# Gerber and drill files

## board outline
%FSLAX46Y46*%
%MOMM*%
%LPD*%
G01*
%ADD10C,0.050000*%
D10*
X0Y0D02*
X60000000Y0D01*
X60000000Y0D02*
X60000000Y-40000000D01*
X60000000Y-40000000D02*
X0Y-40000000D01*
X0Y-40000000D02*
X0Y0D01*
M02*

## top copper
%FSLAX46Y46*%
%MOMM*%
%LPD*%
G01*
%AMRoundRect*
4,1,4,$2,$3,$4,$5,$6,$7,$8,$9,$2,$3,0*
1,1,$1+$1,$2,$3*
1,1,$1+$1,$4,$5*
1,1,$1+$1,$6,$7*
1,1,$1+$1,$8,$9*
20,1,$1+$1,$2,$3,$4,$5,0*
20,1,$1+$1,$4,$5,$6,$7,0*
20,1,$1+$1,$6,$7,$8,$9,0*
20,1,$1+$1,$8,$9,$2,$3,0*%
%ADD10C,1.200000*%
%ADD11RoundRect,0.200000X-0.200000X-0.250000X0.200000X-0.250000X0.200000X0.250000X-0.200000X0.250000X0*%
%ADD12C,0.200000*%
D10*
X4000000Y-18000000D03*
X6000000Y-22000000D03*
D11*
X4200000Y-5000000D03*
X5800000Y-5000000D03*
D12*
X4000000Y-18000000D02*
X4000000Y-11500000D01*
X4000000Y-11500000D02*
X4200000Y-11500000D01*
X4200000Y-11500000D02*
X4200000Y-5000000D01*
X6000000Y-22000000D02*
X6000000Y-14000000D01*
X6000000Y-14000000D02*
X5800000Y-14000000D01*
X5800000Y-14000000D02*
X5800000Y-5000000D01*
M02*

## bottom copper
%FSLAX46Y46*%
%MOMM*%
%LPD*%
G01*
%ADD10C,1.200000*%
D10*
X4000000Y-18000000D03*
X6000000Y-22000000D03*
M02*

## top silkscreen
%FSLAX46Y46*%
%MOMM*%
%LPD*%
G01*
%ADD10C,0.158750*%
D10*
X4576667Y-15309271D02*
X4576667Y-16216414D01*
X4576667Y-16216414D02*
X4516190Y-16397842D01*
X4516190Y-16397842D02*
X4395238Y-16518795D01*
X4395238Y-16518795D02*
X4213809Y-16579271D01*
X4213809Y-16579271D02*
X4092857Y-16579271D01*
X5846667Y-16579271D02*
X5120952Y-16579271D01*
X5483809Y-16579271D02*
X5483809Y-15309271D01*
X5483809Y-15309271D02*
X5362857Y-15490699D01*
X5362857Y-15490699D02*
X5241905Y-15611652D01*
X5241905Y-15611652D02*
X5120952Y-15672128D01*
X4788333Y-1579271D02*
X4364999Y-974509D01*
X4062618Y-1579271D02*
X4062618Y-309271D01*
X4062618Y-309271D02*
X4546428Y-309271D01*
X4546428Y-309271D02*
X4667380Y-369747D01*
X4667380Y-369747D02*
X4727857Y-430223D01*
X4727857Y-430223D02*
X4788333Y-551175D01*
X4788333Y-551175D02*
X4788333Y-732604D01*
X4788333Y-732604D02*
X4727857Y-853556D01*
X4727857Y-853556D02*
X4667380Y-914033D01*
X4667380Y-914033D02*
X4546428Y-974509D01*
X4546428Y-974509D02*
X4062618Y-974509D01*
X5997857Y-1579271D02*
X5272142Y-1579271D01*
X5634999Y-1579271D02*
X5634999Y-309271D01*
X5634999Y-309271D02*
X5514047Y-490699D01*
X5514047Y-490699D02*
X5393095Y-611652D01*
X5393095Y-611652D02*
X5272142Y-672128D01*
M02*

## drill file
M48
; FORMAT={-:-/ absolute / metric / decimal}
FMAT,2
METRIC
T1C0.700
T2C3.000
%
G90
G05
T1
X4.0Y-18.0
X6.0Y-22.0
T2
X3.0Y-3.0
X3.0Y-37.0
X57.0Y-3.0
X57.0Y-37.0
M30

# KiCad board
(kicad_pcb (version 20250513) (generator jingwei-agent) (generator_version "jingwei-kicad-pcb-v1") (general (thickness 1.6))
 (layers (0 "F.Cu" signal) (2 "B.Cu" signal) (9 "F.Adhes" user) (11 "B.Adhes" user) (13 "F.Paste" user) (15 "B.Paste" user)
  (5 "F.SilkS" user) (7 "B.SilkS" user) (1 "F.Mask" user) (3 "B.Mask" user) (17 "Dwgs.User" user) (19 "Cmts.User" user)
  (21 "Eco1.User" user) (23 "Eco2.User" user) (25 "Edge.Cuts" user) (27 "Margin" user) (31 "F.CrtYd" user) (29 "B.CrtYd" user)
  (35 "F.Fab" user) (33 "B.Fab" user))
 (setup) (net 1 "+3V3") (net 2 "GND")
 (gr_line (start 0 0) (end 60 0) (stroke (width 0.05)) (layer "Edge.Cuts"))
 (gr_line (start 60 0) (end 60 40) (stroke (width 0.05)) (layer "Edge.Cuts"))
 (gr_line (start 60 40) (end 0 40) (stroke (width 0.05)) (layer "Edge.Cuts"))
 (gr_line (start 0 40) (end 0 0) (stroke (width 0.05)) (layer "Edge.Cuts"))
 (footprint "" (layer "F.Cu") (at 3 3) (pad "" np_thru_hole circle (at 0 0) (size 3 3) (drill 3) (layers "*.Cu" "*.Mask")))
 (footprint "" (layer "F.Cu") (at 57 3) (pad "" np_thru_hole circle (at 0 0) (size 3 3) (drill 3) (layers "*.Cu" "*.Mask")))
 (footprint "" (layer "F.Cu") (at 3 37) (pad "" np_thru_hole circle (at 0 0) (size 3 3) (drill 3) (layers "*.Cu" "*.Mask")))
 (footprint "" (layer "F.Cu") (at 57 37) (pad "" np_thru_hole circle (at 0 0) (size 3 3) (drill 3) (layers "*.Cu" "*.Mask")))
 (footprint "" (layer "F.Cu") (at 5 20) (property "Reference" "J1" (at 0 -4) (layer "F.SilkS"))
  (pad "1" thru_hole circle (at -1 -2) (size 1.2 1.2) (drill 0.7) (layers "*.Cu" "*.Mask") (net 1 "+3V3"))
  (pad "2" thru_hole circle (at 1 2) (size 1.2 1.2) (drill 0.7) (layers "*.Cu" "*.Mask") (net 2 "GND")))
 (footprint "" (layer "F.Cu") (at 5 5) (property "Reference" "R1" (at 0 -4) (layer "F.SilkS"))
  (pad "1" smd roundrect (at -0.8 0) (size 0.8 0.9) (layers "F.Cu" "F.Paste" "F.Mask") (roundrect_rratio 0.25) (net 1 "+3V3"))
  (pad "2" smd roundrect (at 0.8 0) (size 0.8 0.9) (layers "F.Cu" "F.Paste" "F.Mask") (roundrect_rratio 0.25) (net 2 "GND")))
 (segment (start 4 18) (end 4 11.5) (width 0.2) (layer "F.Cu") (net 1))
 (segment (start 4 11.5) (end 4.2 11.5) (width 0.2) (layer "F.Cu") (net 1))
 (segment (start 4.2 11.5) (end 4.2 5) (width 0.2) (layer "F.Cu") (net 1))
 (segment (start 6 22) (end 6 14) (width 0.2) (layer "F.Cu") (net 2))
 (segment (start 6 14) (end 5.8 14) (width 0.2) (layer "F.Cu") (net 2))
 (segment (start 5.8 14) (end 5.8 5) (width 0.2) (layer "F.Cu") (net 2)))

